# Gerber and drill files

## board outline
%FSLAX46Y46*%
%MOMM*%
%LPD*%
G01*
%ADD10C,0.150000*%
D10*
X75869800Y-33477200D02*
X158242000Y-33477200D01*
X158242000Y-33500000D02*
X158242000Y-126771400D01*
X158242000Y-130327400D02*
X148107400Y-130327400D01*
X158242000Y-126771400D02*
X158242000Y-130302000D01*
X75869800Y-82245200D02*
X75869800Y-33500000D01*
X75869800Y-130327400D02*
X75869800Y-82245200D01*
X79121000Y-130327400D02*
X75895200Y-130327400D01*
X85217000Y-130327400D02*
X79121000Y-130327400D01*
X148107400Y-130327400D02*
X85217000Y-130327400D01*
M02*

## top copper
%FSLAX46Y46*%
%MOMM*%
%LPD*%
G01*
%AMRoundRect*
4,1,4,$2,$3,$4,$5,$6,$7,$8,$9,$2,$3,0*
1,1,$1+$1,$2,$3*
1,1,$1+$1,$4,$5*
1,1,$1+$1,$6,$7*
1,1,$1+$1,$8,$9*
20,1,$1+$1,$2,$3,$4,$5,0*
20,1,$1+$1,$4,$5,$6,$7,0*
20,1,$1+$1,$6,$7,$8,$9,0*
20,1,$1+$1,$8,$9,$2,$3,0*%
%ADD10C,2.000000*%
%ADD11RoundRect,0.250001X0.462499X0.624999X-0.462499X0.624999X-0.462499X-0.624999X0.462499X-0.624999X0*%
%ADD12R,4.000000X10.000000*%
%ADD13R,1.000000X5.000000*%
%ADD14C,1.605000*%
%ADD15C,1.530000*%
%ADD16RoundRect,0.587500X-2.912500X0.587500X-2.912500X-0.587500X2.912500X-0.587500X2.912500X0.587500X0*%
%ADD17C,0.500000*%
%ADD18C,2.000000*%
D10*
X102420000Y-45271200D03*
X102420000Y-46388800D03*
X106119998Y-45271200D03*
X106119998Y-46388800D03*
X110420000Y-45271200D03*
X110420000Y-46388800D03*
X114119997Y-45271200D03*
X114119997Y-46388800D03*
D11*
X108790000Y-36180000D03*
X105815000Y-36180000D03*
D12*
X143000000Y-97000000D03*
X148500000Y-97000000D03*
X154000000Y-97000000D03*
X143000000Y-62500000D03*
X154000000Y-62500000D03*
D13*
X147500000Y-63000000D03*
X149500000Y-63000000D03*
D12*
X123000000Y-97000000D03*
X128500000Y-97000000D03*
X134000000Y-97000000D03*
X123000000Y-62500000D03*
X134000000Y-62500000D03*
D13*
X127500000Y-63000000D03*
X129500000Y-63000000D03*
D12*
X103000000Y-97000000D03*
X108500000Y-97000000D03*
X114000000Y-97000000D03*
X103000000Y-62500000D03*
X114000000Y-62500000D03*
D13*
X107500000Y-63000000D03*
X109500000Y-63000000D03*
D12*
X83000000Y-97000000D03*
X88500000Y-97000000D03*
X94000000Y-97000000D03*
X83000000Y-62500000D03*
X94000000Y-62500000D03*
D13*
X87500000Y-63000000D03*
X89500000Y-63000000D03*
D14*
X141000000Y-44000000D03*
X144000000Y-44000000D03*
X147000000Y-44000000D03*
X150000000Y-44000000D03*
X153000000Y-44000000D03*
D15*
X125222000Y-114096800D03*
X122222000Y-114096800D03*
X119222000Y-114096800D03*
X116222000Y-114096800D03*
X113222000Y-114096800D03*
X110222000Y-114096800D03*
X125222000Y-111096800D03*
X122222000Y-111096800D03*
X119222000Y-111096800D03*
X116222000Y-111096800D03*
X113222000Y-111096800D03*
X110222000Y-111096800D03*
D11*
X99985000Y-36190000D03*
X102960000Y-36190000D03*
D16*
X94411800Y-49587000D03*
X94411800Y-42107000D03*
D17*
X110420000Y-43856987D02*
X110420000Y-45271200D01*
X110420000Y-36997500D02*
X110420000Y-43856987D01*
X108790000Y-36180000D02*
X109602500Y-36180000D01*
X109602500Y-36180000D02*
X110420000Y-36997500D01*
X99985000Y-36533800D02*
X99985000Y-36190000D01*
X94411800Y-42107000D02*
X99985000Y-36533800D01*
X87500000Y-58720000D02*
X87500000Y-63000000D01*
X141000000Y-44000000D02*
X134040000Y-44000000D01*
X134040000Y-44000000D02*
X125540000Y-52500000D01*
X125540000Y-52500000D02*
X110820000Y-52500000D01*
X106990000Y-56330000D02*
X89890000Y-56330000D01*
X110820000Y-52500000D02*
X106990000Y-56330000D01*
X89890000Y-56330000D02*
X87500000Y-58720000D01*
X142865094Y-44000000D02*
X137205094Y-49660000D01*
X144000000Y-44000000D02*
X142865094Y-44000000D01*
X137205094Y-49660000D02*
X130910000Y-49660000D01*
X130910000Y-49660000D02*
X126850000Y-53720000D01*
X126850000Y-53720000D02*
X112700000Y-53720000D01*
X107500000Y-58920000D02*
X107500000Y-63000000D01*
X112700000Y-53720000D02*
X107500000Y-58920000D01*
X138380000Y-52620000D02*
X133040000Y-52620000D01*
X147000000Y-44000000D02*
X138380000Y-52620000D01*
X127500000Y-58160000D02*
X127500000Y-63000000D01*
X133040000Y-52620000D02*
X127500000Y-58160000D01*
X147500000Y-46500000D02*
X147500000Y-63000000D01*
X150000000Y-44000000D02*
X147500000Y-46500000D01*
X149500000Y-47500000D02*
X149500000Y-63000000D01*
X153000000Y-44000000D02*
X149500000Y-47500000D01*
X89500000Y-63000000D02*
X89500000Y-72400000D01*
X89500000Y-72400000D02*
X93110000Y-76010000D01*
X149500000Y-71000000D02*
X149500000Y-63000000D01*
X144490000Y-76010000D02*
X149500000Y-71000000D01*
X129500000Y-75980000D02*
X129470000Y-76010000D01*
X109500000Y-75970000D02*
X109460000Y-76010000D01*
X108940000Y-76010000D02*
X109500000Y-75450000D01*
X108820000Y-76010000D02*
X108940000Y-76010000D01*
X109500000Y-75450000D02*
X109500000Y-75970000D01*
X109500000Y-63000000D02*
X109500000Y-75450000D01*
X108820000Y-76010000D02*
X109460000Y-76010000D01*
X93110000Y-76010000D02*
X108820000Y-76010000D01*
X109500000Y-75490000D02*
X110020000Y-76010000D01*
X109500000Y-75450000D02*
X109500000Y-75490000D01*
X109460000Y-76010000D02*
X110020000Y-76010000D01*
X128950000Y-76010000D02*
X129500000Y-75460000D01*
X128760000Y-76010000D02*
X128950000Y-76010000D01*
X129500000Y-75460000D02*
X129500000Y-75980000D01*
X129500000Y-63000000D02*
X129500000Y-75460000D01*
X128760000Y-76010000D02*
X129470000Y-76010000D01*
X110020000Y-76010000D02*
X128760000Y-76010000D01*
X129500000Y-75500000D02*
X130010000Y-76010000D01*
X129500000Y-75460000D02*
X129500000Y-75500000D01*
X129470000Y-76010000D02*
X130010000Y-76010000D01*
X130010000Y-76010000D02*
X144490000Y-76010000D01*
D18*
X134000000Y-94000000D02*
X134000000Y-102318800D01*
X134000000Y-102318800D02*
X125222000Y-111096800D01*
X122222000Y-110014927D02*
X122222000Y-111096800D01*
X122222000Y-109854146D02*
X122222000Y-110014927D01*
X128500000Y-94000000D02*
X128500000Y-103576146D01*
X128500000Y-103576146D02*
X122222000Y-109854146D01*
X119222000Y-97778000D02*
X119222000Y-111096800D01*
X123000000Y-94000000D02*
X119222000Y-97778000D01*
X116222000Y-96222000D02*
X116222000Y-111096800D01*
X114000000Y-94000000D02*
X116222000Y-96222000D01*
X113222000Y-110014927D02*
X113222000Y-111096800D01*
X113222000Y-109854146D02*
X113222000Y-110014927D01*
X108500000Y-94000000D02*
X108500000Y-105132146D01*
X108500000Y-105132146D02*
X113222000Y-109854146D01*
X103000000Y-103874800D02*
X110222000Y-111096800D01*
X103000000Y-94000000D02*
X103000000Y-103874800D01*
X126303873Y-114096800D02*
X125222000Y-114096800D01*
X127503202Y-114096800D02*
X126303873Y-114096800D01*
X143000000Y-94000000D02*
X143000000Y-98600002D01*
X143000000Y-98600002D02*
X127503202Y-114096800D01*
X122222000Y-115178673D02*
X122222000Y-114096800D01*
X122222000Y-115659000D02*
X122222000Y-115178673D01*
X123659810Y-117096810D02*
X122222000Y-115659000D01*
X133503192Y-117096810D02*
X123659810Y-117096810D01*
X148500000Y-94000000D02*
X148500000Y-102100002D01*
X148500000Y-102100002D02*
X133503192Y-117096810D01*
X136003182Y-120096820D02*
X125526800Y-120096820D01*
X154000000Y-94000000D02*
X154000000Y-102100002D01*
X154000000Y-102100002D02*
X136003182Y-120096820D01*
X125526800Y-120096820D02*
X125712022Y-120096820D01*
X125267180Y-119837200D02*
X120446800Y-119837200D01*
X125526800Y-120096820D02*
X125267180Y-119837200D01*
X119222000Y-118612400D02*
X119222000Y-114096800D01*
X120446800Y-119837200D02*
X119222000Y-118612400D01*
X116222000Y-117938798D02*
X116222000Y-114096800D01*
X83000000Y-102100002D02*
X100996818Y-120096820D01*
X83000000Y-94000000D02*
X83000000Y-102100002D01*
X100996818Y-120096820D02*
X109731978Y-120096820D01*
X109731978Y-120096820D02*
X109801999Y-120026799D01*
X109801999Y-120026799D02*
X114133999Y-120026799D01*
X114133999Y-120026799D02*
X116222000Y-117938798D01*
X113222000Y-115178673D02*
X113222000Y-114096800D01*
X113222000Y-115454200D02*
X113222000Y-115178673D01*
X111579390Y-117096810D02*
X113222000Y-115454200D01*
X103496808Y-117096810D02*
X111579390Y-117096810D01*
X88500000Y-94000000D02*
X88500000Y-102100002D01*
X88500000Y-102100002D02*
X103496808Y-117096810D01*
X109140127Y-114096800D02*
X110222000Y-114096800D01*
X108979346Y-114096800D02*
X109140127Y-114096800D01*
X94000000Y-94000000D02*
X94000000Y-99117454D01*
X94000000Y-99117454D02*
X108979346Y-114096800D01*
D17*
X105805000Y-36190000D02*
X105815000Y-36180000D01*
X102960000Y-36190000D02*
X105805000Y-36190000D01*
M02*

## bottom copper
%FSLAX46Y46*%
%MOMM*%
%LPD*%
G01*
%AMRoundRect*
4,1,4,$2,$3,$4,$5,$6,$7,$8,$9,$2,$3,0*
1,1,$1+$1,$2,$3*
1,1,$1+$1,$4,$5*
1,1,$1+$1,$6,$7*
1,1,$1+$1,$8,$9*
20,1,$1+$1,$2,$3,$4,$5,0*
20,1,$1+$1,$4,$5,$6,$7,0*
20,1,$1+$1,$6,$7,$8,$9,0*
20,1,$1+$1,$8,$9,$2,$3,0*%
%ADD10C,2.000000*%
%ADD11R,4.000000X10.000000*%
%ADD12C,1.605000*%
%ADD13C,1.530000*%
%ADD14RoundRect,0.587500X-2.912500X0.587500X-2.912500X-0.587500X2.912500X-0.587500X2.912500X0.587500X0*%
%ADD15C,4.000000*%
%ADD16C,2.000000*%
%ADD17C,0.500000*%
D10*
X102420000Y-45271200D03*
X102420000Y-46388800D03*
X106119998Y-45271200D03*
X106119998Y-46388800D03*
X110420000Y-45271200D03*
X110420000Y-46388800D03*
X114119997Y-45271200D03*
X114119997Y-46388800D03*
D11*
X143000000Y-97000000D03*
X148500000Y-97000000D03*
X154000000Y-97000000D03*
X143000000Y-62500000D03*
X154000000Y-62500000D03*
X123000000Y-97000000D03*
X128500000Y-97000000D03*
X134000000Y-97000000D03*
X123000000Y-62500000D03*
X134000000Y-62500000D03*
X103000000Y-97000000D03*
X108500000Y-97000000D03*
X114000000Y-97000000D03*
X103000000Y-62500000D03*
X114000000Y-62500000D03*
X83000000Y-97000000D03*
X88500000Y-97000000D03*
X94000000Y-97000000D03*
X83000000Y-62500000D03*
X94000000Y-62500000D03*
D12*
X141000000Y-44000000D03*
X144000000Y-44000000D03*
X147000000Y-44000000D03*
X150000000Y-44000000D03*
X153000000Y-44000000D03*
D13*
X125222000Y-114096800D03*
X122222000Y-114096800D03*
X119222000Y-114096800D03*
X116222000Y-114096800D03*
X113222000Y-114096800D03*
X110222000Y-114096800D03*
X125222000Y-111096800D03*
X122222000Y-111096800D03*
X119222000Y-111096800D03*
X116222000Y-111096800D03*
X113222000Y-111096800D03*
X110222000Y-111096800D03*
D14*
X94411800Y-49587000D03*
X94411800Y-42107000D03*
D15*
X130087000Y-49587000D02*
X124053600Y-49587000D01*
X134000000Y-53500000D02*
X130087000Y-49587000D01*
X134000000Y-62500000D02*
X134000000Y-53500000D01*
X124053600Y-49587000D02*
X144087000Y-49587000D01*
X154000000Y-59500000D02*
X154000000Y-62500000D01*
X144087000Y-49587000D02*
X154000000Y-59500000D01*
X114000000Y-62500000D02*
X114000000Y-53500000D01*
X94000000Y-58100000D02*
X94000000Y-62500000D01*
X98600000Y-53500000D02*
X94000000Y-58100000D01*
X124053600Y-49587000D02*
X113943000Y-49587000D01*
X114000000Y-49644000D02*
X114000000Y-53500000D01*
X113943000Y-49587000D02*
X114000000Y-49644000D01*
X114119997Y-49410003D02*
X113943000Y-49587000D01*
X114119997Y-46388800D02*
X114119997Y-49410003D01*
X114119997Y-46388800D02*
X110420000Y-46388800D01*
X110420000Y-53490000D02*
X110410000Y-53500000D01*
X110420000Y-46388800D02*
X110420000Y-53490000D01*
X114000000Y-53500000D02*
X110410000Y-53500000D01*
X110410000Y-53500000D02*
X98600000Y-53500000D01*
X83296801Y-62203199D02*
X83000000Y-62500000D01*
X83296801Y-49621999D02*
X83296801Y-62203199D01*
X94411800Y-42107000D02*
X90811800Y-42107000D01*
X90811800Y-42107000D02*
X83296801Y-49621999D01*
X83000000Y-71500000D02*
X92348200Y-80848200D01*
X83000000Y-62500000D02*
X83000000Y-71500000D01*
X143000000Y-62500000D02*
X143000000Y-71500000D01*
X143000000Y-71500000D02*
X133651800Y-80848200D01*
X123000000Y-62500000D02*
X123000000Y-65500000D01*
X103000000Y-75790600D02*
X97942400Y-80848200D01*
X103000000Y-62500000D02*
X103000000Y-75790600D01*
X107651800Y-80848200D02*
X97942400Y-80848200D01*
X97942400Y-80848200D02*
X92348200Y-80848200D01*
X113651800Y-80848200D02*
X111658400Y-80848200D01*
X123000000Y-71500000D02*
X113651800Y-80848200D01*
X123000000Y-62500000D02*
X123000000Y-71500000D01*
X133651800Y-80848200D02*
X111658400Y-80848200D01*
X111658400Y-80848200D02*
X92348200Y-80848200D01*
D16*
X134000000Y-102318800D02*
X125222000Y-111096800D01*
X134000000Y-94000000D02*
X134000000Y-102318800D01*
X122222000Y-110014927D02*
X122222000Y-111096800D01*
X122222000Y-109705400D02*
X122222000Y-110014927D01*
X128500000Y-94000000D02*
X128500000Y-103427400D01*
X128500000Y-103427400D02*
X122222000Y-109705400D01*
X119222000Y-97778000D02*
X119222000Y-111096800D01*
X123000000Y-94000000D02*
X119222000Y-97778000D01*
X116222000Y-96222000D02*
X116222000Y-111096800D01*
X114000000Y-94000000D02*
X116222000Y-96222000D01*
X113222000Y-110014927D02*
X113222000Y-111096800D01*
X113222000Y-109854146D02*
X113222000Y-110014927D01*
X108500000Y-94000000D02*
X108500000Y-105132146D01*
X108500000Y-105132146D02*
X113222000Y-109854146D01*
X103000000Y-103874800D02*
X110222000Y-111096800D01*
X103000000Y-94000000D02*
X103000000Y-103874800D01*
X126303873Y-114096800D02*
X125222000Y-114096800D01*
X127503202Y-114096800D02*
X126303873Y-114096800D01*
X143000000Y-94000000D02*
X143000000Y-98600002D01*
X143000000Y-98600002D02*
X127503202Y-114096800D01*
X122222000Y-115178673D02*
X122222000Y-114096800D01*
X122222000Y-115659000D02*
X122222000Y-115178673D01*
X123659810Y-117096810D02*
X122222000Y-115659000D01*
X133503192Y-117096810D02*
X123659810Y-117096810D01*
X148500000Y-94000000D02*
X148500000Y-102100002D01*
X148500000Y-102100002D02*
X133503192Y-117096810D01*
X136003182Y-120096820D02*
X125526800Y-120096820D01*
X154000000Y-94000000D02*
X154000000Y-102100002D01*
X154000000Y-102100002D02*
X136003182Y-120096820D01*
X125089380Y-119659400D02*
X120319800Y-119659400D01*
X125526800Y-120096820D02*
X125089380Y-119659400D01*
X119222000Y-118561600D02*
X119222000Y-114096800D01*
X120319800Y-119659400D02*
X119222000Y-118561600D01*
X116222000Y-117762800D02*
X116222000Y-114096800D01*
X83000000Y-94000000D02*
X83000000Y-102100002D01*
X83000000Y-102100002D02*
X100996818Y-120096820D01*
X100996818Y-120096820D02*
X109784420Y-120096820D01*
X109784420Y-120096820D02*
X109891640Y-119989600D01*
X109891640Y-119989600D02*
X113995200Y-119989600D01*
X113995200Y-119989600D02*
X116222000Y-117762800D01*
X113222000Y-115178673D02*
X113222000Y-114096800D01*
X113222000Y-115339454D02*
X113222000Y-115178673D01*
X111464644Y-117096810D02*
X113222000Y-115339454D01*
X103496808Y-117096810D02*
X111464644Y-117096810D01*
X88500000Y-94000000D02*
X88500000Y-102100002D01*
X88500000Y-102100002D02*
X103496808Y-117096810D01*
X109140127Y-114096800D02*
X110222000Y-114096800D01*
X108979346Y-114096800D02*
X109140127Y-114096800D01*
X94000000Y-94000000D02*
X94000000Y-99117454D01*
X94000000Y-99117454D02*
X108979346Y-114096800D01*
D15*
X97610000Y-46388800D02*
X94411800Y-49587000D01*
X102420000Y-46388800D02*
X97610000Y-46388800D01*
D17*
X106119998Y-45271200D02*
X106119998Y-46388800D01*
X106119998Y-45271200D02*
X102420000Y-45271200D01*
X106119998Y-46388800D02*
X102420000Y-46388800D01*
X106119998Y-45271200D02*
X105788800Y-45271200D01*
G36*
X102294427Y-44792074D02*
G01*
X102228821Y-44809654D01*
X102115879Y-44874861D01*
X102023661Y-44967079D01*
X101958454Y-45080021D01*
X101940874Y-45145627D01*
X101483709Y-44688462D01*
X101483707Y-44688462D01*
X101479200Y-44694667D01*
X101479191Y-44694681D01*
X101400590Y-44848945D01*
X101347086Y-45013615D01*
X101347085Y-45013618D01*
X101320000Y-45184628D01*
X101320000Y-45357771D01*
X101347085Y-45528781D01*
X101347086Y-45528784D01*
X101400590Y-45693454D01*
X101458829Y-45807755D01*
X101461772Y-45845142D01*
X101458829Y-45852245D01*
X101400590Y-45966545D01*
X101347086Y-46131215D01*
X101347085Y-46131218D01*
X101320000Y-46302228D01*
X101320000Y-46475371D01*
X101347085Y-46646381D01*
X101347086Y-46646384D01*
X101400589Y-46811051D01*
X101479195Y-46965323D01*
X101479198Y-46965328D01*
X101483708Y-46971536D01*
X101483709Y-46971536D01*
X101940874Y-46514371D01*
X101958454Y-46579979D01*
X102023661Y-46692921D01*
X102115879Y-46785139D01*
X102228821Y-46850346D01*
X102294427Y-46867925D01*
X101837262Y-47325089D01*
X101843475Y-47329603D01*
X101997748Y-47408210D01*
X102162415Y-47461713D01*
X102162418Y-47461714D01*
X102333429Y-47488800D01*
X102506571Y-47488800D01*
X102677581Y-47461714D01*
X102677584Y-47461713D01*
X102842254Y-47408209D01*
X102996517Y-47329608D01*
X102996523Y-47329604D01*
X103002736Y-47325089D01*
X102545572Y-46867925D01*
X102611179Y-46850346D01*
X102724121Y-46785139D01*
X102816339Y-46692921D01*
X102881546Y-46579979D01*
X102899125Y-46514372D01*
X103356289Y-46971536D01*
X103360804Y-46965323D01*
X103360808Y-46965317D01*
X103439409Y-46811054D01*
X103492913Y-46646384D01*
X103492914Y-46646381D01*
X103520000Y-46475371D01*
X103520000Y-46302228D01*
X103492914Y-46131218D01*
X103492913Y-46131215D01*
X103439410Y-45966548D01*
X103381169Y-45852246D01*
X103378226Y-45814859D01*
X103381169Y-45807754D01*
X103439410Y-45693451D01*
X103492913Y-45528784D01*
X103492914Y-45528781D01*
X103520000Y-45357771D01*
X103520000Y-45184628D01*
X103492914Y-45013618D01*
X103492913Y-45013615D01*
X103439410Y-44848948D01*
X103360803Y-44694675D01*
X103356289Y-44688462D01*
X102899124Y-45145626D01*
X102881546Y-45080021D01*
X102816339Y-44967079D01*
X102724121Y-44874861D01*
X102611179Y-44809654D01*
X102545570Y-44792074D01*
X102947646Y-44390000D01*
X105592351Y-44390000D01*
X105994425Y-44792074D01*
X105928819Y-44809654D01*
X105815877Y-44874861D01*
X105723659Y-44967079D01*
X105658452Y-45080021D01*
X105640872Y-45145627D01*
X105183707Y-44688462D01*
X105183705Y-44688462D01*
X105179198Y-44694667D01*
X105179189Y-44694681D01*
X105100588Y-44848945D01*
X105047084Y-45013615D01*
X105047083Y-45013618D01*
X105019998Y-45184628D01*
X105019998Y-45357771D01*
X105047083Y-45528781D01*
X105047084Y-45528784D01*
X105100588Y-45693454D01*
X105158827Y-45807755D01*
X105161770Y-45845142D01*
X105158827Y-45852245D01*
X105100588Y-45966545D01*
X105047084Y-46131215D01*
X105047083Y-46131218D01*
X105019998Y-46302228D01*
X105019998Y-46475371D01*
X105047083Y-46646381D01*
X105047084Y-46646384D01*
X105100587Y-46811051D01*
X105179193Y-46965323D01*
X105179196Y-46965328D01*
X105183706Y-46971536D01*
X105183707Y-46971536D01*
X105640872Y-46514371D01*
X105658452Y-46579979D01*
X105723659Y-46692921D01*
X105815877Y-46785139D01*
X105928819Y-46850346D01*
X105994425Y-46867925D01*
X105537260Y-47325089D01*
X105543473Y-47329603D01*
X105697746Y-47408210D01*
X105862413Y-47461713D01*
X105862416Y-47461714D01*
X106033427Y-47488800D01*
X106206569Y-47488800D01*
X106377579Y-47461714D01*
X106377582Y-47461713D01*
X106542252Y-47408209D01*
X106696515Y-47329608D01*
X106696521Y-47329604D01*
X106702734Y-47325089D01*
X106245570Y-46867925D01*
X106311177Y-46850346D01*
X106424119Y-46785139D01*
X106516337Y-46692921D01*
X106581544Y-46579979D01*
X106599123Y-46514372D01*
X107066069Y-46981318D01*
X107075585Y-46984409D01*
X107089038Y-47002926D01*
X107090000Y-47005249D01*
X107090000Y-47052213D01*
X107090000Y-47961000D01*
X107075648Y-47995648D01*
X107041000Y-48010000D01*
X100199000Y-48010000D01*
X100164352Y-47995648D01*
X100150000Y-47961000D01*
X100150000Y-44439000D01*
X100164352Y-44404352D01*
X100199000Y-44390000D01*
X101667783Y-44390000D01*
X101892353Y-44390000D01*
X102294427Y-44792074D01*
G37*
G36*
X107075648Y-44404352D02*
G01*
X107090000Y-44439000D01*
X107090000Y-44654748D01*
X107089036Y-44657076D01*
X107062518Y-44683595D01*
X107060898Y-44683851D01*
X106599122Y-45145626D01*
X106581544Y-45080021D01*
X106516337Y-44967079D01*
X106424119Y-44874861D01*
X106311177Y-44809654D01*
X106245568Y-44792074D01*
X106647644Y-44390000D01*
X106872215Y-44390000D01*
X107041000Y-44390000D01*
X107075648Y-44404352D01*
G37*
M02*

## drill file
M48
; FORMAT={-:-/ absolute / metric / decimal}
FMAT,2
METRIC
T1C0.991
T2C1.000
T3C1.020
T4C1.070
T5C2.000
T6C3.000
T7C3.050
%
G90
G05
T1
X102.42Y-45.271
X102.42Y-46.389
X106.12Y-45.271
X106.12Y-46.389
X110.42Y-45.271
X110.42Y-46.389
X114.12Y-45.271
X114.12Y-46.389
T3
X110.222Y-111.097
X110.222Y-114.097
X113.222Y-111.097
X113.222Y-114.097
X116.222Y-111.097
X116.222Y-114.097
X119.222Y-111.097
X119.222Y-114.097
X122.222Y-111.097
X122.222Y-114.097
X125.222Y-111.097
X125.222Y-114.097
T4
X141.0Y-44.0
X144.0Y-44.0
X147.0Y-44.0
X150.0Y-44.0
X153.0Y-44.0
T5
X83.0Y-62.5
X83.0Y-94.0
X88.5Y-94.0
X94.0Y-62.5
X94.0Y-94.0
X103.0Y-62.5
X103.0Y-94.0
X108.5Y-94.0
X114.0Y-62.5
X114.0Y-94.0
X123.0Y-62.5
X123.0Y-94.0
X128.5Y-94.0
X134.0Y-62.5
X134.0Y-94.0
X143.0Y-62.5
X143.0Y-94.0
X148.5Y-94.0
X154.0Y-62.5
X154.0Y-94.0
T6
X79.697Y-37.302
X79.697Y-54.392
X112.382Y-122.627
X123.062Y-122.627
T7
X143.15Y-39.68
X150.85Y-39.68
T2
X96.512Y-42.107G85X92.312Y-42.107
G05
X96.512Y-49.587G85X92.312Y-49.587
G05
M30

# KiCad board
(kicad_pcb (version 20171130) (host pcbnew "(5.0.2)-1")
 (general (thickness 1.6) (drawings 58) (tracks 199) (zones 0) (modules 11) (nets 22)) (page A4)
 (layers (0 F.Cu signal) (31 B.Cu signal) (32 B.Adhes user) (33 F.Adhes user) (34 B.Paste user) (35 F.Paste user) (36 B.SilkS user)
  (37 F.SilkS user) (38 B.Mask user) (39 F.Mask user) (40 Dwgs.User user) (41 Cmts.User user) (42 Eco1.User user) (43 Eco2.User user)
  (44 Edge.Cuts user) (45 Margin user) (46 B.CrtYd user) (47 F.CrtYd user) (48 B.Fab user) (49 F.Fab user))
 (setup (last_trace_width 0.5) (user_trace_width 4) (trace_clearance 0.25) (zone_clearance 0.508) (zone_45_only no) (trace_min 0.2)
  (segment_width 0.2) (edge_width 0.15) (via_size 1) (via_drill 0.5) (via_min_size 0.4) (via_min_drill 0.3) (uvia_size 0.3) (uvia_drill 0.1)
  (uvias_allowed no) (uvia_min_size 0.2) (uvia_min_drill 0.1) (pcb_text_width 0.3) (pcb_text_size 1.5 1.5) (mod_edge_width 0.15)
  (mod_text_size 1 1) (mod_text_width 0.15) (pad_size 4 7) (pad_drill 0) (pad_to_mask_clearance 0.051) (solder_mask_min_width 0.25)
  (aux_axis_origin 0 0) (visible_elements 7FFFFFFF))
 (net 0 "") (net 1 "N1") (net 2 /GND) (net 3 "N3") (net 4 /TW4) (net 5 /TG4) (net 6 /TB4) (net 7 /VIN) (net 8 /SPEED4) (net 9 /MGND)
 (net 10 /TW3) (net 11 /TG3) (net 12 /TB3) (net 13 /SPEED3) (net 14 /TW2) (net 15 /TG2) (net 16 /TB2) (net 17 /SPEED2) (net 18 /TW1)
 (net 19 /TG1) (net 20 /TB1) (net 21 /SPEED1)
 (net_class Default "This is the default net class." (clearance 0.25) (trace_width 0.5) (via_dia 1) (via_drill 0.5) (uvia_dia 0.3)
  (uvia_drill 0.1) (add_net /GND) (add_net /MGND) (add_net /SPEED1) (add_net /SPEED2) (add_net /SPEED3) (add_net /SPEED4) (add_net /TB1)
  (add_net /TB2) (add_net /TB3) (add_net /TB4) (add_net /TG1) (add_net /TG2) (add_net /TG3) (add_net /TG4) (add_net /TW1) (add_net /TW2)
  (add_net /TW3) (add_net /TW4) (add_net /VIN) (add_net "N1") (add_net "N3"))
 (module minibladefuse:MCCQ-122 (layer F.Cu) (at 114.12 45.83 180)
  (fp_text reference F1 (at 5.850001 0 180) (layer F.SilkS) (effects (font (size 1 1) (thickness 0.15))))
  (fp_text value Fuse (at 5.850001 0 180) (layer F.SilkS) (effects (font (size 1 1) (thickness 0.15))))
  (pad 2 thru_hole circle (at 11.7 0.5588 180) (size 2 2) (drill 0.9906) (layers *.Cu *.Mask) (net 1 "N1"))
  (pad 2 thru_hole circle (at 11.7 -0.5588 180) (size 2 2) (drill 0.9906) (layers *.Cu *.Mask) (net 1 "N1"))
  (pad 2 thru_hole circle (at 8.000002 0.5588 180) (size 2 2) (drill 0.9906) (layers *.Cu *.Mask) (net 1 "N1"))
  (pad 2 thru_hole circle (at 8.000002 -0.5588 180) (size 2 2) (drill 0.9906) (layers *.Cu *.Mask) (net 1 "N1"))
  (pad 1 thru_hole circle (at 3.7 0.5588 180) (size 2 2) (drill 0.9906) (layers *.Cu *.Mask) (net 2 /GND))
  (pad 1 thru_hole circle (at 3.7 -0.5588 180) (size 2 2) (drill 0.9906) (layers *.Cu *.Mask) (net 2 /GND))
  (pad 1 thru_hole circle (at 0.000003 0.5588 180) (size 2 2) (drill 0.9906) (layers *.Cu *.Mask) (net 2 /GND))
  (pad 1 thru_hole circle (at 0.000003 -0.5588 180) (size 2 2) (drill 0.9906) (layers *.Cu *.Mask) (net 2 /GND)))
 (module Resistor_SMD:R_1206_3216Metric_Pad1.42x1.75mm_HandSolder (layer F.Cu) (at 107.3025 36.18 180)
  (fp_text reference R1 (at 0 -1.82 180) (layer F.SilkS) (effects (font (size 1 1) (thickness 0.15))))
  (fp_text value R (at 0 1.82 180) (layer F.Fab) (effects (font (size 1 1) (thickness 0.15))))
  (pad 1 smd roundrect (at -1.4875 0 180) (size 1.425 1.75) (layers F.Cu F.Paste F.Mask) (roundrect_rratio 0.175439) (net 2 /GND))
  (pad 2 smd roundrect (at 1.4875 0 180) (size 1.425 1.75) (layers F.Cu F.Paste F.Mask) (roundrect_rratio 0.175439) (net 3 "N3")))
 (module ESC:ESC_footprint (layer F.Cu) (at 140 95)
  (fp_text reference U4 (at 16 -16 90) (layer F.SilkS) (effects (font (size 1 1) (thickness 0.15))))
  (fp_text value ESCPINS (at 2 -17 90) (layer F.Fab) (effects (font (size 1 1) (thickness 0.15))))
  (pad 3 thru_hole rect (at 3 -1) (size 4 10) (drill 2 (offset 0 3)) (layers *.Cu *.Mask) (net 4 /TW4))
  (pad 2 thru_hole rect (at 8.5 -1) (size 4 10) (drill 2 (offset 0 3)) (layers *.Cu *.Mask) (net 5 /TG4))
  (pad 1 thru_hole rect (at 14 -1) (size 4 10) (drill 2 (offset 0 3)) (layers *.Cu *.Mask) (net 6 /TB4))
  (pad 6 thru_hole rect (at 3 -32.5) (size 4 10) (drill 2) (layers *.Cu *.Mask) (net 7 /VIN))
  (pad 7 thru_hole rect (at 14 -32.5) (size 4 10) (drill 2) (layers *.Cu *.Mask) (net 2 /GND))
  (pad 4 smd rect (at 7.5 -32) (size 1 5) (layers F.Cu F.Paste F.Mask) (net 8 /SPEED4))
  (pad 5 smd rect (at 9.5 -32) (size 1 5) (layers F.Cu F.Paste F.Mask) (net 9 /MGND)))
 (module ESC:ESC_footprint (layer F.Cu) (at 120 95)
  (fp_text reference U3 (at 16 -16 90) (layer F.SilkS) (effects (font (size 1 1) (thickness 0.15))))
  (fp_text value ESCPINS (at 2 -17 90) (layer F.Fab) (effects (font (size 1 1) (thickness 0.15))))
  (pad 3 thru_hole rect (at 3 -1) (size 4 10) (drill 2 (offset 0 3)) (layers *.Cu *.Mask) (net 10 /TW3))
  (pad 2 thru_hole rect (at 8.5 -1) (size 4 10) (drill 2 (offset 0 3)) (layers *.Cu *.Mask) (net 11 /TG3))
  (pad 1 thru_hole rect (at 14 -1) (size 4 10) (drill 2 (offset 0 3)) (layers *.Cu *.Mask) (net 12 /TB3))
  (pad 6 thru_hole rect (at 3 -32.5) (size 4 10) (drill 2) (layers *.Cu *.Mask) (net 7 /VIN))
  (pad 7 thru_hole rect (at 14 -32.5) (size 4 10) (drill 2) (layers *.Cu *.Mask) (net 2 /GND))
  (pad 4 smd rect (at 7.5 -32) (size 1 5) (layers F.Cu F.Paste F.Mask) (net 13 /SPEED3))
  (pad 5 smd rect (at 9.5 -32) (size 1 5) (layers F.Cu F.Paste F.Mask) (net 9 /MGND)))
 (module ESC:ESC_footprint (layer F.Cu) (at 100 95)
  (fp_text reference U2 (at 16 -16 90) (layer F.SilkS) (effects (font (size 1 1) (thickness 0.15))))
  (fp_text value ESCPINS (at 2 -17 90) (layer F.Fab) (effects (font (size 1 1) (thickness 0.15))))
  (pad 3 thru_hole rect (at 3 -1) (size 4 10) (drill 2 (offset 0 3)) (layers *.Cu *.Mask) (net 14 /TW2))
  (pad 2 thru_hole rect (at 8.5 -1) (size 4 10) (drill 2 (offset 0 3)) (layers *.Cu *.Mask) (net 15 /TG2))
  (pad 1 thru_hole rect (at 14 -1) (size 4 10) (drill 2 (offset 0 3)) (layers *.Cu *.Mask) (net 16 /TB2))
  (pad 6 thru_hole rect (at 3 -32.5) (size 4 10) (drill 2) (layers *.Cu *.Mask) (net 7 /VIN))
  (pad 7 thru_hole rect (at 14 -32.5) (size 4 10) (drill 2) (layers *.Cu *.Mask) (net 2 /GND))
  (pad 4 smd rect (at 7.5 -32) (size 1 5) (layers F.Cu F.Paste F.Mask) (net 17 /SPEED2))
  (pad 5 smd rect (at 9.5 -32) (size 1 5) (layers F.Cu F.Paste F.Mask) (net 9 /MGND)))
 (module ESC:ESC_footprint (layer F.Cu) (at 80 95)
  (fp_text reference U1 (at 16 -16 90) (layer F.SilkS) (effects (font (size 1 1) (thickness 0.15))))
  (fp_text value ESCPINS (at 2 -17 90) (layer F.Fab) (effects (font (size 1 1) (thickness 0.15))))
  (pad 3 thru_hole rect (at 3 -1) (size 4 10) (drill 2 (offset 0 3)) (layers *.Cu *.Mask) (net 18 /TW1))
  (pad 2 thru_hole rect (at 8.5 -1) (size 4 10) (drill 2 (offset 0 3)) (layers *.Cu *.Mask) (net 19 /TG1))
  (pad 1 thru_hole rect (at 14 -1) (size 4 10) (drill 2 (offset 0 3)) (layers *.Cu *.Mask) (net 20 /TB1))
  (pad 6 thru_hole rect (at 3 -32.5) (size 4 10) (drill 2) (layers *.Cu *.Mask) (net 7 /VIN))
  (pad 7 thru_hole rect (at 14 -32.5) (size 4 10) (drill 2) (layers *.Cu *.Mask) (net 2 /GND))
  (pad 4 smd rect (at 7.5 -32) (size 1 5) (layers F.Cu F.Paste F.Mask) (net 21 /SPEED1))
  (pad 5 smd rect (at 9.5 -32) (size 1 5) (layers F.Cu F.Paste F.Mask) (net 9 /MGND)))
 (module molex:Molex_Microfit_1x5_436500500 (layer F.Cu) (at 141 44 180)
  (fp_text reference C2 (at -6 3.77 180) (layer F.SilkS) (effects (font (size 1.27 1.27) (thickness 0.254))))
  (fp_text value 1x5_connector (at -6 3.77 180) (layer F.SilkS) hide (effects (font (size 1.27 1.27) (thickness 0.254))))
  (pad 1 thru_hole circle (at 0 0 180) (size 1.605 1.605) (drill 1.07) (layers *.Cu *.Mask) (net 21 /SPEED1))
  (pad 2 thru_hole circle (at -3 0 180) (size 1.605 1.605) (drill 1.07) (layers *.Cu *.Mask) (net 17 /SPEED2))
  (pad 3 thru_hole circle (at -6 0 180) (size 1.605 1.605) (drill 1.07) (layers *.Cu *.Mask) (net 13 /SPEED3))
  (pad 4 thru_hole circle (at -9 0 180) (size 1.605 1.605) (drill 1.07) (layers *.Cu *.Mask) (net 8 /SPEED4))
  (pad 5 thru_hole circle (at -12 0 180) (size 1.605 1.605) (drill 1.07) (layers *.Cu *.Mask) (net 9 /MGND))
  (pad MH1 np_thru_hole circle (at -2.15 4.32 180) (size 3.05 0) (drill 3.05) (layers *.Cu *.Mask))
  (pad MH2 np_thru_hole circle (at -9.85 4.32 180) (size 3.05 0) (drill 3.05) (layers *.Cu *.Mask)))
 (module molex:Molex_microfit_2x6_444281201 (layer F.Cu) (at 125.222 114.0968)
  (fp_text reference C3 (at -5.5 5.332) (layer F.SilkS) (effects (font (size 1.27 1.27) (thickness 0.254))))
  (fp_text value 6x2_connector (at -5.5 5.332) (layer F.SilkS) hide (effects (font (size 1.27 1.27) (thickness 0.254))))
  (pad 1 thru_hole circle (at 0 0) (size 1.53 1.53) (drill 1.02) (layers *.Cu *.Mask) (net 4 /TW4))
  (pad 2 thru_hole circle (at -3 0) (size 1.53 1.53) (drill 1.02) (layers *.Cu *.Mask) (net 5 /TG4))
  (pad 3 thru_hole circle (at -6 0) (size 1.53 1.53) (drill 1.02) (layers *.Cu *.Mask) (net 6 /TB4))
  (pad 4 thru_hole circle (at -9 0) (size 1.53 1.53) (drill 1.02) (layers *.Cu *.Mask) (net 18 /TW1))
  (pad 5 thru_hole circle (at -12 0) (size 1.53 1.53) (drill 1.02) (layers *.Cu *.Mask) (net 19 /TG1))
  (pad 6 thru_hole circle (at -15 0) (size 1.53 1.53) (drill 1.02) (layers *.Cu *.Mask) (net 20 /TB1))
  (pad 7 thru_hole circle (at 0 -3) (size 1.53 1.53) (drill 1.02) (layers *.Cu *.Mask) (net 12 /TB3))
  (pad 8 thru_hole circle (at -3 -3) (size 1.53 1.53) (drill 1.02) (layers *.Cu *.Mask) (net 11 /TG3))
  (pad 9 thru_hole circle (at -6 -3) (size 1.53 1.53) (drill 1.02) (layers *.Cu *.Mask) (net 10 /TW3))
  (pad 10 thru_hole circle (at -9 -3) (size 1.53 1.53) (drill 1.02) (layers *.Cu *.Mask) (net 16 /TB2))
  (pad 11 thru_hole circle (at -12 -3) (size 1.53 1.53) (drill 1.02) (layers *.Cu *.Mask) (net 15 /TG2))
  (pad 12 thru_hole circle (at -15 -3) (size 1.53 1.53) (drill 1.02) (layers *.Cu *.Mask) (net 14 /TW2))
  (pad MH1 np_thru_hole circle (at -12.84 8.53) (size 3 0) (drill 3) (layers *.Cu *.Mask))
  (pad MH2 np_thru_hole circle (at -2.16 8.53) (size 3 0) (drill 3) (layers *.Cu *.Mask)))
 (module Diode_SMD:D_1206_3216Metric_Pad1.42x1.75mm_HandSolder (layer F.Cu) (at 101.4725 36.19 180)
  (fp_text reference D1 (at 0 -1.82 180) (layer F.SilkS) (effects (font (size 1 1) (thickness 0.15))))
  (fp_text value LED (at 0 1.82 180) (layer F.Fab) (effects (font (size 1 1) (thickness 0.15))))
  (pad 2 smd roundrect (at 1.4875 0 180) (size 1.425 1.75) (layers F.Cu F.Paste F.Mask) (roundrect_rratio 0.175439) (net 7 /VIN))
  (pad 1 smd roundrect (at -1.4875 0 180) (size 1.425 1.75) (layers F.Cu F.Paste F.Mask) (roundrect_rratio 0.175439) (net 3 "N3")))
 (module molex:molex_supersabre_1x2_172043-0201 (layer F.Cu) (at 94.4118 45.847 270)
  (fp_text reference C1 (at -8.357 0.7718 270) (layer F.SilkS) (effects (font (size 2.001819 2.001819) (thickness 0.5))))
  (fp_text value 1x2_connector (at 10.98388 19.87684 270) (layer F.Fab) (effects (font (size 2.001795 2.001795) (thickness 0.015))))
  (pad 2 thru_hole roundrect (at 3.74 0 270) (size 2.35 7) (drill oval 1 5.2) (layers *.Cu *.Mask) (roundrect_rratio 0.25) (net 1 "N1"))
  (pad 1 thru_hole roundrect (at -3.74 0 270) (size 2.35 7) (drill oval 1 5.2) (layers *.Cu *.Mask) (roundrect_rratio 0.25) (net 7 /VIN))
  (pad None np_thru_hole circle (at -8.545 14.715 270) (size 3 3) (drill 3) (layers *.Cu *.Mask))
  (pad None np_thru_hole circle (at 8.545 14.715 270) (size 3 3) (drill 3) (layers *.Cu *.Mask)))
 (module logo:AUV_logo (layer F.Cu) (at 87.5 125)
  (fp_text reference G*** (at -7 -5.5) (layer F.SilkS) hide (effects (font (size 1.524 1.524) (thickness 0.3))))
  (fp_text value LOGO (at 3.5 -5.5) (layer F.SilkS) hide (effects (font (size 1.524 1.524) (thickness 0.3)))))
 (gr_line (start 75.8698 33.4772) (end 158.242 33.4772) (layer Edge.Cuts) (width 0.15))
 (gr_line (start 158.242 33.5) (end 158.242 126.7714) (layer Edge.Cuts) (width 0.15))
 (gr_line (start 158.242 130.3274) (end 148.1074 130.3274) (layer Edge.Cuts) (width 0.15))
 (gr_line (start 158.242 126.7714) (end 158.242 130.302) (layer Edge.Cuts) (width 0.15))
 (gr_line (start 75.8698 82.2452) (end 75.8698 33.5) (layer Edge.Cuts) (width 0.15))
 (gr_line (start 75.8698 130.3274) (end 75.8698 82.2452) (layer Edge.Cuts) (width 0.15))
 (gr_line (start 79.121 130.3274) (end 75.8952 130.3274) (layer Edge.Cuts) (width 0.15))
 (gr_line (start 85.217 130.3274) (end 79.121 130.3274) (layer Edge.Cuts) (width 0.15))
 (gr_line (start 148.1074 130.3274) (end 85.217 130.3274) (layer Edge.Cuts) (width 0.15))
 (segment (start 130.087 49.587) (end 124.0536 49.587) (width 4) (layer B.Cu) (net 2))
 (segment (start 134 53.5) (end 130.087 49.587) (width 4) (layer B.Cu) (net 2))
 (segment (start 134 62.5) (end 134 53.5) (width 4) (layer B.Cu) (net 2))
 (segment (start 124.0536 49.587) (end 144.087 49.587) (width 4) (layer B.Cu) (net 2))
 (segment (start 154 59.5) (end 154 62.5) (width 4) (layer B.Cu) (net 2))
 (segment (start 144.087 49.587) (end 154 59.5) (width 4) (layer B.Cu) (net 2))
 (segment (start 114 62.5) (end 114 53.5) (width 4) (layer B.Cu) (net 2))
 (segment (start 94 58.1) (end 94 62.5) (width 4) (layer B.Cu) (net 2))
 (segment (start 98.6 53.5) (end 94 58.1) (width 4) (layer B.Cu) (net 2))
 (segment (start 124.0536 49.587) (end 113.943 49.587) (width 4) (layer B.Cu) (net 2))
 (segment (start 114 49.644) (end 114 53.5) (width 4) (layer B.Cu) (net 2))
 (segment (start 113.943 49.587) (end 114 49.644) (width 4) (layer B.Cu) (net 2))
 (segment (start 114.119997 49.410003) (end 113.943 49.587) (width 4) (layer B.Cu) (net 2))
 (segment (start 114.119997 46.3888) (end 114.119997 49.410003) (width 4) (layer B.Cu) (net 2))
 (segment (start 114.119997 46.3888) (end 110.42 46.3888) (width 4) (layer B.Cu) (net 2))
 (segment (start 110.42 53.49) (end 110.41 53.5) (width 4) (layer B.Cu) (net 2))
 (segment (start 110.42 46.3888) (end 110.42 53.49) (width 4) (layer B.Cu) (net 2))
 (segment (start 114 53.5) (end 110.41 53.5) (width 4) (layer B.Cu) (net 2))
 (segment (start 110.41 53.5) (end 98.6 53.5) (width 4) (layer B.Cu) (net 2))
 (segment (start 110.42 43.856987) (end 110.42 45.2712) (width 0.5) (layer F.Cu) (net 2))
 (segment (start 110.42 36.9975) (end 110.42 43.856987) (width 0.5) (layer F.Cu) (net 2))
 (segment (start 108.79 36.18) (end 109.6025 36.18) (width 0.5) (layer F.Cu) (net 2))
 (segment (start 109.6025 36.18) (end 110.42 36.9975) (width 0.5) (layer F.Cu) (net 2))
 (segment (start 83.296801 62.203199) (end 83 62.5) (width 4) (layer B.Cu) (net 7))
 (segment (start 83.296801 49.621999) (end 83.296801 62.203199) (width 4) (layer B.Cu) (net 7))
 (segment (start 94.4118 42.107) (end 90.8118 42.107) (width 4) (layer B.Cu) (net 7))
 (segment (start 90.8118 42.107) (end 83.296801 49.621999) (width 4) (layer B.Cu) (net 7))
 (segment (start 83 71.5) (end 92.3482 80.8482) (width 4) (layer B.Cu) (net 7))
 (segment (start 83 62.5) (end 83 71.5) (width 4) (layer B.Cu) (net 7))
 (segment (start 143 62.5) (end 143 71.5) (width 4) (layer B.Cu) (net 7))
 (segment (start 143 71.5) (end 133.6518 80.8482) (width 4) (layer B.Cu) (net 7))
 (segment (start 123 62.5) (end 123 65.5) (width 4) (layer B.Cu) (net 7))
 (segment (start 103 75.7906) (end 97.9424 80.8482) (width 4) (layer B.Cu) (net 7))
 (segment (start 103 62.5) (end 103 75.7906) (width 4) (layer B.Cu) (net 7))
 (segment (start 107.6518 80.8482) (end 97.9424 80.8482) (width 4) (layer B.Cu) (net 7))
 (segment (start 97.9424 80.8482) (end 92.3482 80.8482) (width 4) (layer B.Cu) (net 7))
 (segment (start 113.6518 80.8482) (end 111.6584 80.8482) (width 4) (layer B.Cu) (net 7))
 (segment (start 123 71.5) (end 113.6518 80.8482) (width 4) (layer B.Cu) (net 7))
 (segment (start 123 62.5) (end 123 71.5) (width 4) (layer B.Cu) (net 7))
 (segment (start 133.6518 80.8482) (end 111.6584 80.8482) (width 4) (layer B.Cu) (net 7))
 (segment (start 111.6584 80.8482) (end 92.3482 80.8482) (width 4) (layer B.Cu) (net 7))
 (segment (start 99.985 36.5338) (end 99.985 36.19) (width 0.5) (layer F.Cu) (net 7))
 (segment (start 94.4118 42.107) (end 99.985 36.5338) (width 0.5) (layer F.Cu) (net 7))
 (segment (start 87.5 58.72) (end 87.5 63) (width 0.5) (layer F.Cu) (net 21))
 (segment (start 141 44) (end 134.04 44) (width 0.5) (layer F.Cu) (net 21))
 (segment (start 134.04 44) (end 125.54 52.5) (width 0.5) (layer F.Cu) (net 21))
 (segment (start 125.54 52.5) (end 110.82 52.5) (width 0.5) (layer F.Cu) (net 21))
 (segment (start 106.99 56.33) (end 89.89 56.33) (width 0.5) (layer F.Cu) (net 21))
 (segment (start 110.82 52.5) (end 106.99 56.33) (width 0.5) (layer F.Cu) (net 21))
 (segment (start 89.89 56.33) (end 87.5 58.72) (width 0.5) (layer F.Cu) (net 21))
 (segment (start 142.865094 44) (end 137.205094 49.66) (width 0.5) (layer F.Cu) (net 17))
 (segment (start 144 44) (end 142.865094 44) (width 0.5) (layer F.Cu) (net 17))
 (segment (start 137.205094 49.66) (end 130.91 49.66) (width 0.5) (layer F.Cu) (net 17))
 (segment (start 130.91 49.66) (end 126.85 53.72) (width 0.5) (layer F.Cu) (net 17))
 (segment (start 126.85 53.72) (end 112.7 53.72) (width 0.5) (layer F.Cu) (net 17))
 (segment (start 107.5 58.92) (end 107.5 63) (width 0.5) (layer F.Cu) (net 17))
 (segment (start 112.7 53.72) (end 107.5 58.92) (width 0.5) (layer F.Cu) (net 17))
 (segment (start 138.38 52.62) (end 133.04 52.62) (width 0.5) (layer F.Cu) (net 13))
 (segment (start 147 44) (end 138.38 52.62) (width 0.5) (layer F.Cu) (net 13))
 (segment (start 127.5 58.16) (end 127.5 63) (width 0.5) (layer F.Cu) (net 13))
 (segment (start 133.04 52.62) (end 127.5 58.16) (width 0.5) (layer F.Cu) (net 13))
 (segment (start 147.5 46.5) (end 147.5 63) (width 0.5) (layer F.Cu) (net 8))
 (segment (start 150 44) (end 147.5 46.5) (width 0.5) (layer F.Cu) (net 8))
 (segment (start 149.5 47.5) (end 149.5 63) (width 0.5) (layer F.Cu) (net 9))
 (segment (start 153 44) (end 149.5 47.5) (width 0.5) (layer F.Cu) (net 9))
 (segment (start 89.5 63) (end 89.5 72.4) (width 0.5) (layer F.Cu) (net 9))
 (segment (start 89.5 72.4) (end 93.11 76.01) (width 0.5) (layer F.Cu) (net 9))
 (segment (start 149.5 71) (end 149.5 63) (width 0.5) (layer F.Cu) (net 9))
 (segment (start 144.49 76.01) (end 149.5 71) (width 0.5) (layer F.Cu) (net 9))
 (segment (start 129.5 75.98) (end 129.47 76.01) (width 0.5) (layer F.Cu) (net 9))
 (segment (start 109.5 75.97) (end 109.46 76.01) (width 0.5) (layer F.Cu) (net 9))
 (segment (start 108.94 76.01) (end 109.5 75.45) (width 0.5) (layer F.Cu) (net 9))
 (segment (start 108.82 76.01) (end 108.94 76.01) (width 0.5) (layer F.Cu) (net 9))
 (segment (start 109.5 75.45) (end 109.5 75.97) (width 0.5) (layer F.Cu) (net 9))
 (segment (start 109.5 63) (end 109.5 75.45) (width 0.5) (layer F.Cu) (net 9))
 (segment (start 108.82 76.01) (end 109.46 76.01) (width 0.5) (layer F.Cu) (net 9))
 (segment (start 93.11 76.01) (end 108.82 76.01) (width 0.5) (layer F.Cu) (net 9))
 (segment (start 109.5 75.49) (end 110.02 76.01) (width 0.5) (layer F.Cu) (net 9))
 (segment (start 109.5 75.45) (end 109.5 75.49) (width 0.5) (layer F.Cu) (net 9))
 (segment (start 109.46 76.01) (end 110.02 76.01) (width 0.5) (layer F.Cu) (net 9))
 (segment (start 128.95 76.01) (end 129.5 75.46) (width 0.5) (layer F.Cu) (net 9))
 (segment (start 128.76 76.01) (end 128.95 76.01) (width 0.5) (layer F.Cu) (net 9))
 (segment (start 129.5 75.46) (end 129.5 75.98) (width 0.5) (layer F.Cu) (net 9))
 (segment (start 129.5 63) (end 129.5 75.46) (width 0.5) (layer F.Cu) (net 9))
 (segment (start 128.76 76.01) (end 129.47 76.01) (width 0.5) (layer F.Cu) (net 9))
 (segment (start 110.02 76.01) (end 128.76 76.01) (width 0.5) (layer F.Cu) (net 9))
 (segment (start 129.5 75.5) (end 130.01 76.01) (width 0.5) (layer F.Cu) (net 9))
 (segment (start 129.5 75.46) (end 129.5 75.5) (width 0.5) (layer F.Cu) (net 9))
 (segment (start 129.47 76.01) (end 130.01 76.01) (width 0.5) (layer F.Cu) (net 9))
 (segment (start 130.01 76.01) (end 144.49 76.01) (width 0.5) (layer F.Cu) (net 9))
 (segment (start 134 94) (end 134 102.3188) (width 2) (layer F.Cu) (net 12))
 (segment (start 134 102.3188) (end 125.222 111.0968) (width 2) (layer F.Cu) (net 12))
 (segment (start 134 102.3188) (end 125.222 111.0968) (width 2) (layer B.Cu) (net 12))
 (segment (start 134 94) (end 134 102.3188) (width 2) (layer B.Cu) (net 12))
 (segment (start 122.222 110.014927) (end 122.222 111.0968) (width 2) (layer B.Cu) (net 11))
 (segment (start 122.222 109.7054) (end 122.222 110.014927) (width 2) (layer B.Cu) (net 11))
 (segment (start 128.5 94) (end 128.5 103.4274) (width 2) (layer B.Cu) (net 11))
 (segment (start 128.5 103.4274) (end 122.222 109.7054) (width 2) (layer B.Cu) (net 11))
 (segment (start 122.222 110.014927) (end 122.222 111.0968) (width 2) (layer F.Cu) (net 11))
 (segment (start 122.222 109.854146) (end 122.222 110.014927) (width 2) (layer F.Cu) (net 11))
 (segment (start 128.5 94) (end 128.5 103.576146) (width 2) (layer F.Cu) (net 11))
 (segment (start 128.5 103.576146) (end 122.222 109.854146) (width 2) (layer F.Cu) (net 11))
 (segment (start 119.222 97.778) (end 119.222 111.0968) (width 2) (layer F.Cu) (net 10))
 (segment (start 123 94) (end 119.222 97.778) (width 2) (layer F.Cu) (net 10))
 (segment (start 119.222 97.778) (end 119.222 111.0968) (width 2) (layer B.Cu) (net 10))
 (segment (start 123 94) (end 119.222 97.778) (width 2) (layer B.Cu) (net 10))
 (segment (start 116.222 96.222) (end 116.222 111.0968) (width 2) (layer F.Cu) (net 16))
 (segment (start 114 94) (end 116.222 96.222) (width 2) (layer F.Cu) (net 16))
 (segment (start 116.222 96.222) (end 116.222 111.0968) (width 2) (layer B.Cu) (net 16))
 (segment (start 114 94) (end 116.222 96.222) (width 2) (layer B.Cu) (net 16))
 (segment (start 113.222 110.014927) (end 113.222 111.0968) (width 2) (layer B.Cu) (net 15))
 (segment (start 113.222 109.854146) (end 113.222 110.014927) (width 2) (layer B.Cu) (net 15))
 (segment (start 108.5 94) (end 108.5 105.132146) (width 2) (layer B.Cu) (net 15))
 (segment (start 108.5 105.132146) (end 113.222 109.854146) (width 2) (layer B.Cu) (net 15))
 (segment (start 113.222 110.014927) (end 113.222 111.0968) (width 2) (layer F.Cu) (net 15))
 (segment (start 113.222 109.854146) (end 113.222 110.014927) (width 2) (layer F.Cu) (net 15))
 (segment (start 108.5 94) (end 108.5 105.132146) (width 2) (layer F.Cu) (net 15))
 (segment (start 108.5 105.132146) (end 113.222 109.854146) (width 2) (layer F.Cu) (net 15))
 (segment (start 103 103.8748) (end 110.222 111.0968) (width 2) (layer F.Cu) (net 14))
 (segment (start 103 94) (end 103 103.8748) (width 2) (layer F.Cu) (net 14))
 (segment (start 103 103.8748) (end 110.222 111.0968) (width 2) (layer B.Cu) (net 14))
 (segment (start 103 94) (end 103 103.8748) (width 2) (layer B.Cu) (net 14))
 (segment (start 126.303873 114.0968) (end 125.222 114.0968) (width 2) (layer F.Cu) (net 4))
 (segment (start 127.503202 114.0968) (end 126.303873 114.0968) (width 2) (layer F.Cu) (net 4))
 (segment (start 143 94) (end 143 98.600002) (width 2) (layer F.Cu) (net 4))
 (segment (start 143 98.600002) (end 127.503202 114.0968) (width 2) (layer F.Cu) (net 4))
 (segment (start 126.303873 114.0968) (end 125.222 114.0968) (width 2) (layer B.Cu) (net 4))
 (segment (start 127.503202 114.0968) (end 126.303873 114.0968) (width 2) (layer B.Cu) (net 4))
 (segment (start 143 94) (end 143 98.600002) (width 2) (layer B.Cu) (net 4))
 (segment (start 143 98.600002) (end 127.503202 114.0968) (width 2) (layer B.Cu) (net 4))
 (segment (start 122.222 115.178673) (end 122.222 114.0968) (width 2) (layer F.Cu) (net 5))
 (segment (start 122.222 115.659) (end 122.222 115.178673) (width 2) (layer F.Cu) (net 5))
 (segment (start 123.65981 117.09681) (end 122.222 115.659) (width 2) (layer F.Cu) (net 5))
 (segment (start 133.503192 117.09681) (end 123.65981 117.09681) (width 2) (layer F.Cu) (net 5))
 (segment (start 148.5 94) (end 148.5 102.100002) (width 2) (layer F.Cu) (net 5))
 (segment (start 148.5 102.100002) (end 133.503192 117.09681) (width 2) (layer F.Cu) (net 5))
 (segment (start 122.222 115.178673) (end 122.222 114.0968) (width 2) (layer B.Cu) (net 5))
 (segment (start 122.222 115.659) (end 122.222 115.178673) (width 2) (layer B.Cu) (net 5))
 (segment (start 123.65981 117.09681) (end 122.222 115.659) (width 2) (layer B.Cu) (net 5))
 (segment (start 133.503192 117.09681) (end 123.65981 117.09681) (width 2) (layer B.Cu) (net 5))
 (segment (start 148.5 94) (end 148.5 102.100002) (width 2) (layer B.Cu) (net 5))
 (segment (start 148.5 102.100002) (end 133.503192 117.09681) (width 2) (layer B.Cu) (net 5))
 (segment (start 136.003182 120.09682) (end 125.5268 120.09682) (width 2) (layer F.Cu) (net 6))
 (segment (start 154 94) (end 154 102.100002) (width 2) (layer F.Cu) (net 6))
 (segment (start 154 102.100002) (end 136.003182 120.09682) (width 2) (layer F.Cu) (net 6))
 (segment (start 125.5268 120.09682) (end 125.712022 120.09682) (width 2) (layer F.Cu) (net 6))
 (segment (start 125.26718 119.8372) (end 120.4468 119.8372) (width 2) (layer F.Cu) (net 6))
 (segment (start 125.5268 120.09682) (end 125.26718 119.8372) (width 2) (layer F.Cu) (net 6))
 (segment (start 119.222 118.6124) (end 119.222 114.0968) (width 2) (layer F.Cu) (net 6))
 (segment (start 120.4468 119.8372) (end 119.222 118.6124) (width 2) (layer F.Cu) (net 6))
 (segment (start 136.003182 120.09682) (end 125.5268 120.09682) (width 2) (layer B.Cu) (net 6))
 (segment (start 154 94) (end 154 102.100002) (width 2) (layer B.Cu) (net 6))
 (segment (start 154 102.100002) (end 136.003182 120.09682) (width 2) (layer B.Cu) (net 6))
 (segment (start 125.08938 119.6594) (end 120.3198 119.6594) (width 2) (layer B.Cu) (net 6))
 (segment (start 125.5268 120.09682) (end 125.08938 119.6594) (width 2) (layer B.Cu) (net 6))
 (segment (start 119.222 118.5616) (end 119.222 114.0968) (width 2) (layer B.Cu) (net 6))
 (segment (start 120.3198 119.6594) (end 119.222 118.5616) (width 2) (layer B.Cu) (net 6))
 (segment (start 116.222 117.938798) (end 116.222 114.0968) (width 2) (layer F.Cu) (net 18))
 (segment (start 83 102.100002) (end 100.996818 120.09682) (width 2) (layer F.Cu) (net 18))
 (segment (start 83 94) (end 83 102.100002) (width 2) (layer F.Cu) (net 18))
 (segment (start 100.996818 120.09682) (end 109.731978 120.09682) (width 2) (layer F.Cu) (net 18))
 (segment (start 109.731978 120.09682) (end 109.801999 120.026799) (width 2) (layer F.Cu) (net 18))
 (segment (start 109.801999 120.026799) (end 114.133999 120.026799) (width 2) (layer F.Cu) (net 18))
 (segment (start 114.133999 120.026799) (end 116.222 117.938798) (width 2) (layer F.Cu) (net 18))
 (segment (start 116.222 117.7628) (end 116.222 114.0968) (width 2) (layer B.Cu) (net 18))
 (segment (start 83 94) (end 83 102.100002) (width 2) (layer B.Cu) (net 18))
 (segment (start 83 102.100002) (end 100.996818 120.09682) (width 2) (layer B.Cu) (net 18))
 (segment (start 100.996818 120.09682) (end 109.78442 120.09682) (width 2) (layer B.Cu) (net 18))
 (segment (start 109.78442 120.09682) (end 109.89164 119.9896) (width 2) (layer B.Cu) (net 18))
 (segment (start 109.89164 119.9896) (end 113.9952 119.9896) (width 2) (layer B.Cu) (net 18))
 (segment (start 113.9952 119.9896) (end 116.222 117.7628) (width 2) (layer B.Cu) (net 18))
 (segment (start 113.222 115.178673) (end 113.222 114.0968) (width 2) (layer F.Cu) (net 19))
 (segment (start 113.222 115.4542) (end 113.222 115.178673) (width 2) (layer F.Cu) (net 19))
 (segment (start 111.57939 117.09681) (end 113.222 115.4542) (width 2) (layer F.Cu) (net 19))
 (segment (start 103.496808 117.09681) (end 111.57939 117.09681) (width 2) (layer F.Cu) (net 19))
 (segment (start 88.5 94) (end 88.5 102.100002) (width 2) (layer F.Cu) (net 19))
 (segment (start 88.5 102.100002) (end 103.496808 117.09681) (width 2) (layer F.Cu) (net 19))
 (segment (start 113.222 115.178673) (end 113.222 114.0968) (width 2) (layer B.Cu) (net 19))
 (segment (start 113.222 115.339454) (end 113.222 115.178673) (width 2) (layer B.Cu) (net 19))
 (segment (start 111.464644 117.09681) (end 113.222 115.339454) (width 2) (layer B.Cu) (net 19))
 (segment (start 103.496808 117.09681) (end 111.464644 117.09681) (width 2) (layer B.Cu) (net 19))
 (segment (start 88.5 94) (end 88.5 102.100002) (width 2) (layer B.Cu) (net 19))
 (segment (start 88.5 102.100002) (end 103.496808 117.09681) (width 2) (layer B.Cu) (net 19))
 (segment (start 109.140127 114.0968) (end 110.222 114.0968) (width 2) (layer F.Cu) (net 20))
 (segment (start 108.979346 114.0968) (end 109.140127 114.0968) (width 2) (layer F.Cu) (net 20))
 (segment (start 94 94) (end 94 99.117454) (width 2) (layer F.Cu) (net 20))
 (segment (start 94 99.117454) (end 108.979346 114.0968) (width 2) (layer F.Cu) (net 20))
 (segment (start 109.140127 114.0968) (end 110.222 114.0968) (width 2) (layer B.Cu) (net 20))
 (segment (start 108.979346 114.0968) (end 109.140127 114.0968) (width 2) (layer B.Cu) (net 20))
 (segment (start 94 94) (end 94 99.117454) (width 2) (layer B.Cu) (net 20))
 (segment (start 94 99.117454) (end 108.979346 114.0968) (width 2) (layer B.Cu) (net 20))
 (segment (start 105.805 36.19) (end 105.815 36.18) (width 0.5) (layer F.Cu) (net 3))
 (segment (start 102.96 36.19) (end 105.805 36.19) (width 0.5) (layer F.Cu) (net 3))
 (segment (start 97.61 46.3888) (end 94.4118 49.587) (width 4) (layer B.Cu) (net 1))
 (segment (start 102.42 46.3888) (end 97.61 46.3888) (width 4) (layer B.Cu) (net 1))
 (segment (start 106.119998 45.2712) (end 106.119998 46.3888) (width 0.5) (layer B.Cu) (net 1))
 (segment (start 106.119998 45.2712) (end 102.42 45.2712) (width 0.5) (layer B.Cu) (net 1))
 (segment (start 106.119998 46.3888) (end 102.42 46.3888) (width 0.5) (layer B.Cu) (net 1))
 (segment (start 106.119998 45.2712) (end 105.7888 45.2712) (width 0.5) (layer B.Cu) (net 1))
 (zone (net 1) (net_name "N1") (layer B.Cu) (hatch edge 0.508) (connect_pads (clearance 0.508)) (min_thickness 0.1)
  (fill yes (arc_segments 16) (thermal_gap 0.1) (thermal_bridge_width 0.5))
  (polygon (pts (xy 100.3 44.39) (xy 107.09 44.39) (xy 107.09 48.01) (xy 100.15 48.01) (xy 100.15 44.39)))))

